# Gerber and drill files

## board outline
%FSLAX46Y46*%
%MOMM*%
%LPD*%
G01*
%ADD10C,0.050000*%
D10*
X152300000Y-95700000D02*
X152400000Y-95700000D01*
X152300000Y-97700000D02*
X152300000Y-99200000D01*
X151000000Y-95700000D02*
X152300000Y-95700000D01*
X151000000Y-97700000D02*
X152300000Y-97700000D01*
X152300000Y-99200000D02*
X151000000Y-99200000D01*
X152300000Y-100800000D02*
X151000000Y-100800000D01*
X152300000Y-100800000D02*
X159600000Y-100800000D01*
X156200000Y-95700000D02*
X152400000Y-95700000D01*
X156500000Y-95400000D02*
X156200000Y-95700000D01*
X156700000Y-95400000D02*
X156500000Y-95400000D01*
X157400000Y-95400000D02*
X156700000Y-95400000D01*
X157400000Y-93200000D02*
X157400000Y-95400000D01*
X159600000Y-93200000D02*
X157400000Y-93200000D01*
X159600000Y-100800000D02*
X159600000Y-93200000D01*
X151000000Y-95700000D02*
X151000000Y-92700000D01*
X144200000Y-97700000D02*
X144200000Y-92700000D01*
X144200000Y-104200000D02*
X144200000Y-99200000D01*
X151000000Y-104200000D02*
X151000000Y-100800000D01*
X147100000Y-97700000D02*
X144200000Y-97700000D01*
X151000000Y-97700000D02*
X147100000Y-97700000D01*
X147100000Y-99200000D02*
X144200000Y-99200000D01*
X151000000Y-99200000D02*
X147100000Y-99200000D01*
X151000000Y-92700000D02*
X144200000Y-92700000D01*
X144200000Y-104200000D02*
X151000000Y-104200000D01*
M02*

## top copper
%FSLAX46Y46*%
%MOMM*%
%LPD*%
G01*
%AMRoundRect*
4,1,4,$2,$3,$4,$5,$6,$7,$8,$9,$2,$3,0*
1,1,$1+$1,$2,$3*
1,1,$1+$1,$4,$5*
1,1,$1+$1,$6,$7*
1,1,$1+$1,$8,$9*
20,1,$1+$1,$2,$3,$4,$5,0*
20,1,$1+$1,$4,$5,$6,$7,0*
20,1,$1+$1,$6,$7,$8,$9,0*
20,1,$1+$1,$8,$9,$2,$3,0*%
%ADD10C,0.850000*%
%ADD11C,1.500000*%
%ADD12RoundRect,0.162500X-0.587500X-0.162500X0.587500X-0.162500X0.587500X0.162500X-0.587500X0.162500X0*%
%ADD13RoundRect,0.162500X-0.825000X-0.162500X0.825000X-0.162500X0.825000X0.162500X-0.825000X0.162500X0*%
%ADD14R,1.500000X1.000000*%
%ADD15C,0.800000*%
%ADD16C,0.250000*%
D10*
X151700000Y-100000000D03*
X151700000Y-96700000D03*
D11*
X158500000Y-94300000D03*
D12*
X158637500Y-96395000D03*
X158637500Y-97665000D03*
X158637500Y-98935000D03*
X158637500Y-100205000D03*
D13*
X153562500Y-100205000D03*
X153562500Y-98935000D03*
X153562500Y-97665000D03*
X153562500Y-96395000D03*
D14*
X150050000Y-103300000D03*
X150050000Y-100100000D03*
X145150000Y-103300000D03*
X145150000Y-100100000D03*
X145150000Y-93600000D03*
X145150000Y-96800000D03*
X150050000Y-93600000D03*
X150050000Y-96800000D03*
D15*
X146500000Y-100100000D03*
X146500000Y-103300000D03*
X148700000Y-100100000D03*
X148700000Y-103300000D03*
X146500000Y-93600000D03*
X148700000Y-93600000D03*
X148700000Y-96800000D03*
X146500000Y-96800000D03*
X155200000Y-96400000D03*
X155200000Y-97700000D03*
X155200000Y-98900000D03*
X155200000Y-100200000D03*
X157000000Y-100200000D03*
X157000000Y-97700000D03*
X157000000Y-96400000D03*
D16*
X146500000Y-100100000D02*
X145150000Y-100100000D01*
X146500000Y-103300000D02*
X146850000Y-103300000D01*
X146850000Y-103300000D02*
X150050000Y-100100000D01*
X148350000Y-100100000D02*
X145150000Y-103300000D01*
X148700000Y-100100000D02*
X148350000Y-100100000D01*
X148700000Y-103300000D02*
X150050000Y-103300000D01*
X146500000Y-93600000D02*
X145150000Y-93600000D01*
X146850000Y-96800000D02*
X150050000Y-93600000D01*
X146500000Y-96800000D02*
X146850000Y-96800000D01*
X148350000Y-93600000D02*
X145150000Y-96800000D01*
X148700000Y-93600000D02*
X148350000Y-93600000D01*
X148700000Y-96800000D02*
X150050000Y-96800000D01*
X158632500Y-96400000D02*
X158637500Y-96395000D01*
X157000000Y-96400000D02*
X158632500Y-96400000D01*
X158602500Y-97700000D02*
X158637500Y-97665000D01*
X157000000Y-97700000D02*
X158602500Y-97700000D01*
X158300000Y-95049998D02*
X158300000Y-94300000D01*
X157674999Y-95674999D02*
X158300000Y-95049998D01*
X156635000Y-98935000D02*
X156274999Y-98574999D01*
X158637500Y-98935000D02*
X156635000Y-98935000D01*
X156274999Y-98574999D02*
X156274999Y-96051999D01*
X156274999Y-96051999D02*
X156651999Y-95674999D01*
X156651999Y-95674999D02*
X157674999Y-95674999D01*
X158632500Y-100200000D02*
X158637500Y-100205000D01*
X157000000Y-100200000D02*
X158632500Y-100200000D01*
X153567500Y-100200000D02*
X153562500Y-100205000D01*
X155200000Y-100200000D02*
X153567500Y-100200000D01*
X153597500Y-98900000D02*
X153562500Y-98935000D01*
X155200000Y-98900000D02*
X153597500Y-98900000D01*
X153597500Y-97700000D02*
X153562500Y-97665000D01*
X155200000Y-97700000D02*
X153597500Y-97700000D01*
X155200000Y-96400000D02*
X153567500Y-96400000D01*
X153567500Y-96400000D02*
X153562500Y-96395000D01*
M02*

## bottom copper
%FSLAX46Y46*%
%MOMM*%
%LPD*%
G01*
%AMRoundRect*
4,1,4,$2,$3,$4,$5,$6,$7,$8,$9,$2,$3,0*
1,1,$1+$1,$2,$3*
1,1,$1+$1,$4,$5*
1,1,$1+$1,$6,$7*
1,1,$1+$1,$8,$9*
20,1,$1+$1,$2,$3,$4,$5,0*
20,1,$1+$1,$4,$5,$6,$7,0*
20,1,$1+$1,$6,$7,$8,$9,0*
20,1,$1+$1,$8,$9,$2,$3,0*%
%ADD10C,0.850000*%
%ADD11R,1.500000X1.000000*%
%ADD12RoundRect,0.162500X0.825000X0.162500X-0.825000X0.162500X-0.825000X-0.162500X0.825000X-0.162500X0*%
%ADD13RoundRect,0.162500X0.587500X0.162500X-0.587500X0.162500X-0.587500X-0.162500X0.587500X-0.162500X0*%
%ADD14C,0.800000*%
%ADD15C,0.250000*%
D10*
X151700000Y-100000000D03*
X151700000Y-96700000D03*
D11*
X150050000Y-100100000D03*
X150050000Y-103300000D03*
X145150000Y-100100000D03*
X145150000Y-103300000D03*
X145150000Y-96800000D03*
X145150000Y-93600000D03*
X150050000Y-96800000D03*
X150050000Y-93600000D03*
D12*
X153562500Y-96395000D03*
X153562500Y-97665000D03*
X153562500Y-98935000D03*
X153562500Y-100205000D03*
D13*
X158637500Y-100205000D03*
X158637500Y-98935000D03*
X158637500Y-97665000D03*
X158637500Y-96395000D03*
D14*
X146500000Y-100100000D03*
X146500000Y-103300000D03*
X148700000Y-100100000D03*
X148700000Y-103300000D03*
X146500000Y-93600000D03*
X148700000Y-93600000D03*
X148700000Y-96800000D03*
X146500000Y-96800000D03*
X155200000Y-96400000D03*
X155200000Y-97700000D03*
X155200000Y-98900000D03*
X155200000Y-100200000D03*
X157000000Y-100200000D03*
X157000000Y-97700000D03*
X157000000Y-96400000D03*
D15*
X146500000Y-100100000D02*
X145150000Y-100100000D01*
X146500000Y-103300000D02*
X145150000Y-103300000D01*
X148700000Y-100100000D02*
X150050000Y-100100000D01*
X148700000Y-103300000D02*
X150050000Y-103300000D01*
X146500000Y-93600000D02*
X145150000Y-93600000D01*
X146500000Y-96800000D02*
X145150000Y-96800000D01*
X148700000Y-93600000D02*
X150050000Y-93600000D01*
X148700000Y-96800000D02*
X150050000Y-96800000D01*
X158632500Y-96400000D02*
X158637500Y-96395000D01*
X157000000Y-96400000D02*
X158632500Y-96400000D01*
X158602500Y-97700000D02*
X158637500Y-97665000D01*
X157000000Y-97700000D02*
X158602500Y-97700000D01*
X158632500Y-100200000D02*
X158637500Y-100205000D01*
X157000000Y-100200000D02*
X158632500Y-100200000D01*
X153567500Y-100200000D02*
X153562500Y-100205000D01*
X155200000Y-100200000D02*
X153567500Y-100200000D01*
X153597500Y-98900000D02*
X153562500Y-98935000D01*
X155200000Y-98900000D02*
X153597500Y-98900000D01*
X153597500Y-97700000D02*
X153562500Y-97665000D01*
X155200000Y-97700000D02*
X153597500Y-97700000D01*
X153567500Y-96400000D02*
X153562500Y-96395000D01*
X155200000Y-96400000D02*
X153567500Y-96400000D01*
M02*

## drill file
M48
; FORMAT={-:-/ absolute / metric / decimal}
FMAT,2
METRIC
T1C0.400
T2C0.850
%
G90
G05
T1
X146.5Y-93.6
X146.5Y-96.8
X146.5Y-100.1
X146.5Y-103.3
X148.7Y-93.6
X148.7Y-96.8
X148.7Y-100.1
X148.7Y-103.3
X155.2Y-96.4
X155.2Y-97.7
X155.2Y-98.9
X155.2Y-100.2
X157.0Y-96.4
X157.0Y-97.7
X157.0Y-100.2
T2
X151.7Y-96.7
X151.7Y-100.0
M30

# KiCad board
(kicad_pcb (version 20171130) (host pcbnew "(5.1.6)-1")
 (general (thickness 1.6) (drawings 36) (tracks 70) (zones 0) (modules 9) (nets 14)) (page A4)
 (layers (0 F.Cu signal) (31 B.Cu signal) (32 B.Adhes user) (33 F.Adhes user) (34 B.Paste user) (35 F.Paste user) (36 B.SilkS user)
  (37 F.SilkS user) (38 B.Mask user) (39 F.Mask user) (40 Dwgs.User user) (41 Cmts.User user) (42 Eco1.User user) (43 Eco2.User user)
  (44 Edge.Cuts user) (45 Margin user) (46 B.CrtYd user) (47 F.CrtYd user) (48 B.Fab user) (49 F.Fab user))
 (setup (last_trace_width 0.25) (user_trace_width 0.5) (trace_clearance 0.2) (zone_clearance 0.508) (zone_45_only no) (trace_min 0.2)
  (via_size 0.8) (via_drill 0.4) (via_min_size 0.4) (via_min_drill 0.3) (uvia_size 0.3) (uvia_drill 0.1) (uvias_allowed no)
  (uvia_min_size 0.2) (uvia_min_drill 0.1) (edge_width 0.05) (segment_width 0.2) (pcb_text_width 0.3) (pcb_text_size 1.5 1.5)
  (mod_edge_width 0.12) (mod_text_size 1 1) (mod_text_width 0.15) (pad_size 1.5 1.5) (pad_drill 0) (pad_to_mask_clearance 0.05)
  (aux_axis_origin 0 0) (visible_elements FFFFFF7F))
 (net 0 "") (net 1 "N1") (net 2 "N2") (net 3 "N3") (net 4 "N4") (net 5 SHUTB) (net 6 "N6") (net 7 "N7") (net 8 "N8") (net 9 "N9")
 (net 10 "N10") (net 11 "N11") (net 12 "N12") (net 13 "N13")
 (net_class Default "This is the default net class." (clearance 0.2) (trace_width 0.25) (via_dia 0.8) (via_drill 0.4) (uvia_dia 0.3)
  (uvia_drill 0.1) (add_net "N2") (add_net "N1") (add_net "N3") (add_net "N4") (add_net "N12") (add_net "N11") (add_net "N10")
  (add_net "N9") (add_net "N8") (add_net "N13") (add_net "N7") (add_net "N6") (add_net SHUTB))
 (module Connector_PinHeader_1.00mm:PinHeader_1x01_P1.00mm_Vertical (layer F.Cu) (at 151.7 100)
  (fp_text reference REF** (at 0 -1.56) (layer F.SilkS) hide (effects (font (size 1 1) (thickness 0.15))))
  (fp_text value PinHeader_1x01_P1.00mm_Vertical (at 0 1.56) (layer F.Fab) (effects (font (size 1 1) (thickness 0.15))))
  (pad 1 thru_hole circle (at 0 0) (size 0.85 0.85) (drill 0.85) (layers *.Cu *.Mask)))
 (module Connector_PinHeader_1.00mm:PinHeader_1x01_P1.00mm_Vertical (layer F.Cu) (at 151.7 96.7)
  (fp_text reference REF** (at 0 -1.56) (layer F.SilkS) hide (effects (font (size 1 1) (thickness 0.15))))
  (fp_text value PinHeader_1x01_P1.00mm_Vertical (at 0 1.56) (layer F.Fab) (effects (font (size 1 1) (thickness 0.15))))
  (pad 1 thru_hole circle (at 0 0) (size 0.85 0.85) (drill 0.85) (layers *.Cu *.Mask)))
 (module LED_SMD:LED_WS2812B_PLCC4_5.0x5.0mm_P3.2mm (layer B.Cu) (at 147.6 101.7)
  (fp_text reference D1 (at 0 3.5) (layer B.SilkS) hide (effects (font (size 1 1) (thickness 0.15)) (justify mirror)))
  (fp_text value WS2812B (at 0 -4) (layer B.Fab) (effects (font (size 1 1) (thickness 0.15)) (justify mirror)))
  (pad 3 smd rect (at 2.45 -1.6) (size 1.5 1) (layers B.Cu B.Paste B.Mask))
  (pad 4 smd rect (at 2.45 1.6) (size 1.5 1) (layers B.Cu B.Paste B.Mask))
  (pad 2 smd rect (at -2.45 -1.6) (size 1.5 1) (layers B.Cu B.Paste B.Mask))
  (pad 1 smd rect (at -2.45 1.6) (size 1.5 1) (layers B.Cu B.Paste B.Mask)))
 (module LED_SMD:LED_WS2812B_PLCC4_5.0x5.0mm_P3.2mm (layer B.Cu) (at 147.6 95.2)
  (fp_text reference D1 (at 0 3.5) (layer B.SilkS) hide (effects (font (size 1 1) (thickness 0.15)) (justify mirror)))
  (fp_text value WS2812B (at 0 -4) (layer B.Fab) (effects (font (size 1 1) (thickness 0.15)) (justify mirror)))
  (pad 1 smd rect (at -2.45 1.6) (size 1.5 1) (layers B.Cu B.Paste B.Mask) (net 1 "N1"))
  (pad 2 smd rect (at -2.45 -1.6) (size 1.5 1) (layers B.Cu B.Paste B.Mask) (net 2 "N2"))
  (pad 4 smd rect (at 2.45 1.6) (size 1.5 1) (layers B.Cu B.Paste B.Mask) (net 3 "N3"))
  (pad 3 smd rect (at 2.45 -1.6) (size 1.5 1) (layers B.Cu B.Paste B.Mask) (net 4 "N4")))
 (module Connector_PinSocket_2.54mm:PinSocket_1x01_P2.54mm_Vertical (layer F.Cu) (at 158.3 94.3)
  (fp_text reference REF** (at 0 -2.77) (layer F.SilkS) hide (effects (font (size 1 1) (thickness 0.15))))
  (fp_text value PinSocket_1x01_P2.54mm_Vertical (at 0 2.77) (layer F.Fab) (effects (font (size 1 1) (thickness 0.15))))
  (pad 1 smd circle (at 0.2 0) (size 1.5 1.5) (layers F.Cu F.Paste F.Mask) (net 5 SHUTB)))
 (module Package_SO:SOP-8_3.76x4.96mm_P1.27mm (layer F.Cu) (at 156.1 98.3)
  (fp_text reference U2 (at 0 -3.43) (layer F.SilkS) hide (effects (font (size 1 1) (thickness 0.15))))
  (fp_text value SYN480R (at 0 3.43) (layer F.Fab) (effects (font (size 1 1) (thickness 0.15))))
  (pad 8 smd roundrect (at 2.5375 -1.905) (size 1.5 0.65) (layers F.Cu F.Paste F.Mask) (roundrect_rratio 0.25) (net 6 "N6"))
  (pad 7 smd roundrect (at 2.5375 -0.635) (size 1.5 0.65) (layers F.Cu F.Paste F.Mask) (roundrect_rratio 0.25) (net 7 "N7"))
  (pad 6 smd roundrect (at 2.5375 0.635) (size 1.5 0.65) (layers F.Cu F.Paste F.Mask) (roundrect_rratio 0.25) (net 5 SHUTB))
  (pad 5 smd roundrect (at 2.5375 1.905) (size 1.5 0.65) (layers F.Cu F.Paste F.Mask) (roundrect_rratio 0.25) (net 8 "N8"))
  (pad 4 smd roundrect (at -2.5375 1.905) (size 1.975 0.65) (layers F.Cu F.Paste F.Mask) (roundrect_rratio 0.25) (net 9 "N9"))
  (pad 3 smd roundrect (at -2.5375 0.635) (size 1.975 0.65) (layers F.Cu F.Paste F.Mask) (roundrect_rratio 0.25) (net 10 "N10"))
  (pad 2 smd roundrect (at -2.5375 -0.635) (size 1.975 0.65) (layers F.Cu F.Paste F.Mask) (roundrect_rratio 0.25) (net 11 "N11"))
  (pad 1 smd roundrect (at -2.5375 -1.905) (size 1.975 0.65) (layers F.Cu F.Paste F.Mask) (roundrect_rratio 0.25) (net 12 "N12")))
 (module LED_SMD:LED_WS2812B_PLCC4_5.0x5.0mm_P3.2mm (layer F.Cu) (at 147.6 101.7)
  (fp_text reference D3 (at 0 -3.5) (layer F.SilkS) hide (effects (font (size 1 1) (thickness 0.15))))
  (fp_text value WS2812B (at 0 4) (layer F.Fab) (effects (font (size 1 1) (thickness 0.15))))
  (pad 3 smd rect (at 2.45 1.6) (size 1.5 1) (layers F.Cu F.Paste F.Mask))
  (pad 4 smd rect (at 2.45 -1.6) (size 1.5 1) (layers F.Cu F.Paste F.Mask))
  (pad 2 smd rect (at -2.45 1.6) (size 1.5 1) (layers F.Cu F.Paste F.Mask))
  (pad 1 smd rect (at -2.45 -1.6) (size 1.5 1) (layers F.Cu F.Paste F.Mask)))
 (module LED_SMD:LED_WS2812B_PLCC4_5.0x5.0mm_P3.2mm (layer F.Cu) (at 147.6 95.2)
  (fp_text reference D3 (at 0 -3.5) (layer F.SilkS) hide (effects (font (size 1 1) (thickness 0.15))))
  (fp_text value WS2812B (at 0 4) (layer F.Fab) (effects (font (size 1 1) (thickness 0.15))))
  (pad 1 smd rect (at -2.45 -1.6) (size 1.5 1) (layers F.Cu F.Paste F.Mask) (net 2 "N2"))
  (pad 2 smd rect (at -2.45 1.6) (size 1.5 1) (layers F.Cu F.Paste F.Mask) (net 4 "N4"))
  (pad 4 smd rect (at 2.45 -1.6) (size 1.5 1) (layers F.Cu F.Paste F.Mask) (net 1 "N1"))
  (pad 3 smd rect (at 2.45 1.6) (size 1.5 1) (layers F.Cu F.Paste F.Mask) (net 3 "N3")))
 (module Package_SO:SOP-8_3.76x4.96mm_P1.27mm (layer B.Cu) (at 156.1 98.3 180)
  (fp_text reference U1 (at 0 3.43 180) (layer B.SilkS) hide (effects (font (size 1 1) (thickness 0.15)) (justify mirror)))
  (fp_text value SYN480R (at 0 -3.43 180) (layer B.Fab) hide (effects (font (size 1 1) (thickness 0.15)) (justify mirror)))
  (pad 4 smd roundrect (at 2.5375 1.905 180) (size 1.975 0.65) (layers B.Cu B.Paste B.Mask) (roundrect_rratio 0.25) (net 12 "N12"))
  (pad 3 smd roundrect (at 2.5375 0.635 180) (size 1.975 0.65) (layers B.Cu B.Paste B.Mask) (roundrect_rratio 0.25) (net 11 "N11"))
  (pad 2 smd roundrect (at 2.5375 -0.635 180) (size 1.975 0.65) (layers B.Cu B.Paste B.Mask) (roundrect_rratio 0.25) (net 10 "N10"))
  (pad 1 smd roundrect (at 2.5375 -1.905 180) (size 1.975 0.65) (layers B.Cu B.Paste B.Mask) (roundrect_rratio 0.25) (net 9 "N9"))
  (pad 5 smd roundrect (at -2.5375 -1.905 180) (size 1.5 0.65) (layers B.Cu B.Paste B.Mask) (roundrect_rratio 0.25) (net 8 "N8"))
  (pad 6 smd roundrect (at -2.5375 -0.635 180) (size 1.5 0.65) (layers B.Cu B.Paste B.Mask) (roundrect_rratio 0.25) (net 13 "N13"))
  (pad 7 smd roundrect (at -2.5375 0.635 180) (size 1.5 0.65) (layers B.Cu B.Paste B.Mask) (roundrect_rratio 0.25) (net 7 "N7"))
  (pad 8 smd roundrect (at -2.5375 1.905 180) (size 1.5 0.65) (layers B.Cu B.Paste B.Mask) (roundrect_rratio 0.25) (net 6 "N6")))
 (gr_line (start 152.3 95.7) (end 152.4 95.7) (layer Edge.Cuts) (width 0.05))
 (gr_line (start 152.3 97.7) (end 152.3 99.2) (layer Edge.Cuts) (width 0.05))
 (gr_line (start 151 95.7) (end 152.3 95.7) (layer Edge.Cuts) (width 0.05))
 (gr_line (start 151 97.7) (end 152.3 97.7) (layer Edge.Cuts) (width 0.05))
 (gr_line (start 152.3 99.2) (end 151 99.2) (layer Edge.Cuts) (width 0.05))
 (gr_line (start 152.3 100.8) (end 151 100.8) (layer Edge.Cuts) (width 0.05))
 (gr_line (start 152.3 100.8) (end 159.6 100.8) (layer Edge.Cuts) (width 0.05))
 (gr_line (start 156.2 95.7) (end 152.4 95.7) (layer Edge.Cuts) (width 0.05))
 (gr_line (start 156.5 95.4) (end 156.2 95.7) (layer Edge.Cuts) (width 0.05))
 (gr_line (start 156.7 95.4) (end 156.5 95.4) (layer Edge.Cuts) (width 0.05))
 (gr_line (start 157.4 95.4) (end 156.7 95.4) (layer Edge.Cuts) (width 0.05))
 (gr_line (start 157.4 93.2) (end 157.4 95.4) (layer Edge.Cuts) (width 0.05))
 (gr_line (start 159.6 93.2) (end 157.4 93.2) (layer Edge.Cuts) (width 0.05))
 (gr_line (start 159.6 100.8) (end 159.6 93.2) (layer Edge.Cuts) (width 0.05))
 (gr_line (start 151 95.7) (end 151 92.7) (layer Edge.Cuts) (width 0.05))
 (gr_line (start 144.2 97.7) (end 144.2 92.7) (layer Edge.Cuts) (width 0.05))
 (gr_line (start 144.2 104.2) (end 144.2 99.2) (layer Edge.Cuts) (width 0.05))
 (gr_line (start 151 104.2) (end 151 100.8) (layer Edge.Cuts) (width 0.05))
 (gr_line (start 147.1 97.7) (end 144.2 97.7) (layer Edge.Cuts) (width 0.05))
 (gr_line (start 151 97.7) (end 147.1 97.7) (layer Edge.Cuts) (width 0.05))
 (gr_line (start 147.1 99.2) (end 144.2 99.2) (layer Edge.Cuts) (width 0.05))
 (gr_line (start 151 99.2) (end 147.1 99.2) (layer Edge.Cuts) (width 0.05))
 (gr_line (start 151 92.7) (end 144.2 92.7) (layer Edge.Cuts) (width 0.05))
 (gr_line (start 144.2 104.2) (end 151 104.2) (layer Edge.Cuts) (width 0.05))
 (via (at 146.5 100.1) (size 0.8) (drill 0.4) (layers F.Cu B.Cu) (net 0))
 (segment (start 146.5 100.1) (end 145.15 100.1) (width 0.25) (layer F.Cu) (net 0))
 (segment (start 146.5 100.1) (end 145.15 100.1) (width 0.25) (layer B.Cu) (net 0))
 (via (at 146.5 103.3) (size 0.8) (drill 0.4) (layers F.Cu B.Cu) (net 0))
 (segment (start 146.5 103.3) (end 146.85 103.3) (width 0.25) (layer F.Cu) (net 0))
 (segment (start 146.5 103.3) (end 145.15 103.3) (width 0.25) (layer B.Cu) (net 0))
 (segment (start 146.85 103.3) (end 150.05 100.1) (width 0.25) (layer F.Cu) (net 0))
 (via (at 148.7 100.1) (size 0.8) (drill 0.4) (layers F.Cu B.Cu) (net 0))
 (segment (start 148.35 100.1) (end 145.15 103.3) (width 0.25) (layer F.Cu) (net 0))
 (segment (start 148.7 100.1) (end 148.35 100.1) (width 0.25) (layer F.Cu) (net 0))
 (segment (start 148.7 100.1) (end 150.05 100.1) (width 0.25) (layer B.Cu) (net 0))
 (via (at 148.7 103.3) (size 0.8) (drill 0.4) (layers F.Cu B.Cu) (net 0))
 (segment (start 148.7 103.3) (end 150.05 103.3) (width 0.25) (layer F.Cu) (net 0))
 (segment (start 148.7 103.3) (end 150.05 103.3) (width 0.25) (layer B.Cu) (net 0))
 (via (at 146.5 93.6) (size 0.8) (drill 0.4) (layers F.Cu B.Cu) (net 2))
 (segment (start 146.5 93.6) (end 145.15 93.6) (width 0.25) (layer F.Cu) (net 2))
 (segment (start 146.5 93.6) (end 145.15 93.6) (width 0.25) (layer B.Cu) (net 2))
 (via (at 148.7 93.6) (size 0.8) (drill 0.4) (layers F.Cu B.Cu) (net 4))
 (via (at 148.7 96.8) (size 0.8) (drill 0.4) (layers F.Cu B.Cu) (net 3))
 (via (at 146.5 96.8) (size 0.8) (drill 0.4) (layers F.Cu B.Cu) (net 1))
 (segment (start 146.85 96.8) (end 150.05 93.6) (width 0.25) (layer F.Cu) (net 1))
 (segment (start 146.5 96.8) (end 146.85 96.8) (width 0.25) (layer F.Cu) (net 1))
 (segment (start 146.5 96.8) (end 145.15 96.8) (width 0.25) (layer B.Cu) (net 1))
 (segment (start 148.35 93.6) (end 145.15 96.8) (width 0.25) (layer F.Cu) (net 4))
 (segment (start 148.7 93.6) (end 148.35 93.6) (width 0.25) (layer F.Cu) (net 4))
 (segment (start 148.7 93.6) (end 150.05 93.6) (width 0.25) (layer B.Cu) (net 4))
 (segment (start 148.7 96.8) (end 150.05 96.8) (width 0.25) (layer F.Cu) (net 3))
 (segment (start 148.7 96.8) (end 150.05 96.8) (width 0.25) (layer B.Cu) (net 3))
 (via (at 155.2 96.4) (size 0.8) (drill 0.4) (layers F.Cu B.Cu) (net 12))
 (via (at 155.2 97.7) (size 0.8) (drill 0.4) (layers F.Cu B.Cu) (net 11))
 (via (at 155.2 98.9) (size 0.8) (drill 0.4) (layers F.Cu B.Cu) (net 10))
 (via (at 155.2 100.2) (size 0.8) (drill 0.4) (layers F.Cu B.Cu) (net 9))
 (via (at 157 100.2) (size 0.8) (drill 0.4) (layers F.Cu B.Cu) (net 8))
 (via (at 157 97.7) (size 0.8) (drill 0.4) (layers F.Cu B.Cu) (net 7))
 (via (at 157 96.4) (size 0.8) (drill 0.4) (layers F.Cu B.Cu) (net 6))
 (segment (start 158.6325 96.4) (end 158.6375 96.395) (width 0.25) (layer F.Cu) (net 6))
 (segment (start 157 96.4) (end 158.6325 96.4) (width 0.25) (layer F.Cu) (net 6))
 (segment (start 158.6325 96.4) (end 158.6375 96.395) (width 0.25) (layer B.Cu) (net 6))
 (segment (start 157 96.4) (end 158.6325 96.4) (width 0.25) (layer B.Cu) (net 6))
 (segment (start 158.6025 97.7) (end 158.6375 97.665) (width 0.25) (layer F.Cu) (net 7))
 (segment (start 157 97.7) (end 158.6025 97.7) (width 0.25) (layer F.Cu) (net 7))
 (segment (start 158.6025 97.7) (end 158.6375 97.665) (width 0.25) (layer B.Cu) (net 7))
 (segment (start 157 97.7) (end 158.6025 97.7) (width 0.25) (layer B.Cu) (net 7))
 (segment (start 158.3 95.049998) (end 158.3 94.3) (width 0.25) (layer F.Cu) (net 5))
 (segment (start 157.674999 95.674999) (end 158.3 95.049998) (width 0.25) (layer F.Cu) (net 5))
 (segment (start 156.635 98.935) (end 156.274999 98.574999) (width 0.25) (layer F.Cu) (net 5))
 (segment (start 158.6375 98.935) (end 156.635 98.935) (width 0.25) (layer F.Cu) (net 5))
 (segment (start 156.274999 98.574999) (end 156.274999 96.051999) (width 0.25) (layer F.Cu) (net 5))
 (segment (start 156.274999 96.051999) (end 156.651999 95.674999) (width 0.25) (layer F.Cu) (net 5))
 (segment (start 156.651999 95.674999) (end 157.674999 95.674999) (width 0.25) (layer F.Cu) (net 5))
 (segment (start 158.6325 100.2) (end 158.6375 100.205) (width 0.25) (layer F.Cu) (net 8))
 (segment (start 157 100.2) (end 158.6325 100.2) (width 0.25) (layer F.Cu) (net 8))
 (segment (start 158.6325 100.2) (end 158.6375 100.205) (width 0.25) (layer B.Cu) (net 8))
 (segment (start 157 100.2) (end 158.6325 100.2) (width 0.25) (layer B.Cu) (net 8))
 (segment (start 153.5675 100.2) (end 153.5625 100.205) (width 0.25) (layer F.Cu) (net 9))
 (segment (start 155.2 100.2) (end 153.5675 100.2) (width 0.25) (layer F.Cu) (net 9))
 (segment (start 153.5675 100.2) (end 153.5625 100.205) (width 0.25) (layer B.Cu) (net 9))
 (segment (start 155.2 100.2) (end 153.5675 100.2) (width 0.25) (layer B.Cu) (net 9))
 (segment (start 153.5975 98.9) (end 153.5625 98.935) (width 0.25) (layer F.Cu) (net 10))
 (segment (start 155.2 98.9) (end 153.5975 98.9) (width 0.25) (layer F.Cu) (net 10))
 (segment (start 153.5975 98.9) (end 153.5625 98.935) (width 0.25) (layer B.Cu) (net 10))
 (segment (start 155.2 98.9) (end 153.5975 98.9) (width 0.25) (layer B.Cu) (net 10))
 (segment (start 153.5975 97.7) (end 153.5625 97.665) (width 0.25) (layer F.Cu) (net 11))
 (segment (start 155.2 97.7) (end 153.5975 97.7) (width 0.25) (layer F.Cu) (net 11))
 (segment (start 153.5975 97.7) (end 153.5625 97.665) (width 0.25) (layer B.Cu) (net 11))
 (segment (start 155.2 97.7) (end 153.5975 97.7) (width 0.25) (layer B.Cu) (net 11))
 (segment (start 155.2 96.4) (end 153.5675 96.4) (width 0.25) (layer F.Cu) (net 12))
 (segment (start 153.5675 96.4) (end 153.5625 96.395) (width 0.25) (layer F.Cu) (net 12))
 (segment (start 153.5675 96.4) (end 153.5625 96.395) (width 0.25) (layer B.Cu) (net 12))
 (segment (start 155.2 96.4) (end 153.5675 96.4) (width 0.25) (layer B.Cu) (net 12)))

